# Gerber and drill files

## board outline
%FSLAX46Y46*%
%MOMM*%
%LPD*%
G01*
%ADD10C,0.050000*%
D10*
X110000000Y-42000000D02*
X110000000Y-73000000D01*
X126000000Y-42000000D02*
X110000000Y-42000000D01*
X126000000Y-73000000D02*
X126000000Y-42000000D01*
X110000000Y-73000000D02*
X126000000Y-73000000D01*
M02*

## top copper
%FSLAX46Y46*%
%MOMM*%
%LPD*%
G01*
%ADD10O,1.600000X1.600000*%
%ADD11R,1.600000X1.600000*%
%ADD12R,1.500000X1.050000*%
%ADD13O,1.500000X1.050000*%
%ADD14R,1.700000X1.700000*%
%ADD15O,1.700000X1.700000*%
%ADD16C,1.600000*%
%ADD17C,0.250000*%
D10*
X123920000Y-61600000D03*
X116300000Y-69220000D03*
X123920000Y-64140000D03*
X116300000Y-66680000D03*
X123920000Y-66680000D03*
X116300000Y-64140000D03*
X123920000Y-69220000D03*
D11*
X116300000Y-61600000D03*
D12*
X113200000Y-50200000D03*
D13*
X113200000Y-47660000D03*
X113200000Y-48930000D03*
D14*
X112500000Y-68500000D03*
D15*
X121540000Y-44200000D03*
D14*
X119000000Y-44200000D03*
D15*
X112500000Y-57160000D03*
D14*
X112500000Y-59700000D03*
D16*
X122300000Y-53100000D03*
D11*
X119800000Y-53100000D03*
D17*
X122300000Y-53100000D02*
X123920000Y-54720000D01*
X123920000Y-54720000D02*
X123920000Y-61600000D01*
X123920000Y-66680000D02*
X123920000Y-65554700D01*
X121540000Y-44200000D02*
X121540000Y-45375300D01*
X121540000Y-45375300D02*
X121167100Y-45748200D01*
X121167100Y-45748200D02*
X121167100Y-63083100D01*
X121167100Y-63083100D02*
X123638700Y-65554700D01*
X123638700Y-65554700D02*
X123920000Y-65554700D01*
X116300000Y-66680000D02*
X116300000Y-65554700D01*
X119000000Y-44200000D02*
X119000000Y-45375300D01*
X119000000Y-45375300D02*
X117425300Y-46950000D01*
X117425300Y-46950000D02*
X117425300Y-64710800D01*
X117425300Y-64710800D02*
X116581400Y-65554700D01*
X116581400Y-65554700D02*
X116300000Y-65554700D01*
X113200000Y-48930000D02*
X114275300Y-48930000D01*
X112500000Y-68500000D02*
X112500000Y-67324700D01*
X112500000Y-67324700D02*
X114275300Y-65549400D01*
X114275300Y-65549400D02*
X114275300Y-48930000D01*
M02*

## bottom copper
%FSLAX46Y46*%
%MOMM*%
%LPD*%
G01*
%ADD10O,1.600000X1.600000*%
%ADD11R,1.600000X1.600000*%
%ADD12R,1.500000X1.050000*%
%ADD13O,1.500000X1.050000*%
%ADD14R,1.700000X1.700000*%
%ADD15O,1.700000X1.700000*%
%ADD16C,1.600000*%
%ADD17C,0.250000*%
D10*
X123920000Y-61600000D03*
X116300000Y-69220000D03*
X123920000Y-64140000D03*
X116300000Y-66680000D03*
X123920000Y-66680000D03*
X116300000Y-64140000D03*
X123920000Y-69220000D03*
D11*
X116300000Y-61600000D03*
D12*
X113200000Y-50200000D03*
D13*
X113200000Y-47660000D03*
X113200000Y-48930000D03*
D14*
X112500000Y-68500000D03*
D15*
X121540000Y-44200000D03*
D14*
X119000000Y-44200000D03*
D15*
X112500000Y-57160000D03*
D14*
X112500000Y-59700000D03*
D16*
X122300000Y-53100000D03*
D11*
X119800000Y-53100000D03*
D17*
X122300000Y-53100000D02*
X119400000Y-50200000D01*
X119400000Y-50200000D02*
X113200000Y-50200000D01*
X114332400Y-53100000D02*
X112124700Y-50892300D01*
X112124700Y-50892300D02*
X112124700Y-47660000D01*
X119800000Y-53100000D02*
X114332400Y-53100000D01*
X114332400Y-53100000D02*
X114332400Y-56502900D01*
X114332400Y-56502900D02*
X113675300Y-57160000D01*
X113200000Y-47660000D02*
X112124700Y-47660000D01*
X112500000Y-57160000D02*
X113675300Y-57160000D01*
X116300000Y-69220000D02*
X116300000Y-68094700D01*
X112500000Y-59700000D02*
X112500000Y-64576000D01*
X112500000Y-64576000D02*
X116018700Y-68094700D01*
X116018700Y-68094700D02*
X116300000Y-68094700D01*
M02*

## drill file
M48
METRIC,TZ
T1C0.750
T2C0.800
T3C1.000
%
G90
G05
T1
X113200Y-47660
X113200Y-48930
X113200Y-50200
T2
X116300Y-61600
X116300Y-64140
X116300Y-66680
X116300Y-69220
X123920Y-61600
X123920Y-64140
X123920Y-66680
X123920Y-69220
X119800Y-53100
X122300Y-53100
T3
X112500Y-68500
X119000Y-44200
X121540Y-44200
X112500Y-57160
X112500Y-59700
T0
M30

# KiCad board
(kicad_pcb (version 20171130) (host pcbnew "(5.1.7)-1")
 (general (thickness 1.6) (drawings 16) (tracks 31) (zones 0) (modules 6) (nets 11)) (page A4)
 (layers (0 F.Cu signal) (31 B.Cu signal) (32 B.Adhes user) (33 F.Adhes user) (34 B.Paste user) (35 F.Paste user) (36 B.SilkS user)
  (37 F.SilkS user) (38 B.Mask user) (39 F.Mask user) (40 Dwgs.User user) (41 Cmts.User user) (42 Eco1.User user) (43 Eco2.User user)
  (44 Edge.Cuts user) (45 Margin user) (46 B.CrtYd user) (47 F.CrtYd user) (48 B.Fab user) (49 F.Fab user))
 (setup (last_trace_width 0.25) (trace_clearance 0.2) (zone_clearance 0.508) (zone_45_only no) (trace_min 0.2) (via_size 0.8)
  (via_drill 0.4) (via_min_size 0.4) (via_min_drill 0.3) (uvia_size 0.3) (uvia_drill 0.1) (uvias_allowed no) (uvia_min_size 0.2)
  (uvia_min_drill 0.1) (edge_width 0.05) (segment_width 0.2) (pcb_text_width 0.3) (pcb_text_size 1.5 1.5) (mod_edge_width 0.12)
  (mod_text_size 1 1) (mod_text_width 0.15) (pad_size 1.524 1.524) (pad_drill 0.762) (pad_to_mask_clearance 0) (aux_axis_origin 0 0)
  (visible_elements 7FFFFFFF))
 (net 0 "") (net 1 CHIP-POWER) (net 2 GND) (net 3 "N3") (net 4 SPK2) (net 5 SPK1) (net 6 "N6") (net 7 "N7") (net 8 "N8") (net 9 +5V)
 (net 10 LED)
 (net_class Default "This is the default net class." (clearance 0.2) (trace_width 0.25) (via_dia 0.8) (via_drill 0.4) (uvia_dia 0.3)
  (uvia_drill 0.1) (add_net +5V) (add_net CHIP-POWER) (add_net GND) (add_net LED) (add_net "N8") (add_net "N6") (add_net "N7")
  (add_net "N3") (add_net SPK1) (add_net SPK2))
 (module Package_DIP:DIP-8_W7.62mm (layer F.Cu) (at 116.3 61.6)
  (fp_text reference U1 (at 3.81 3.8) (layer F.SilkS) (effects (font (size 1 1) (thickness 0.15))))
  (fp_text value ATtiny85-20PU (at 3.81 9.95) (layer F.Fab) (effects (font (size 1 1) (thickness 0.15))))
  (pad 8 thru_hole oval (at 7.62 0) (size 1.6 1.6) (drill 0.8) (layers *.Cu *.Mask) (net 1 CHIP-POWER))
  (pad 4 thru_hole oval (at 0 7.62) (size 1.6 1.6) (drill 0.8) (layers *.Cu *.Mask) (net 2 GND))
  (pad 7 thru_hole oval (at 7.62 2.54) (size 1.6 1.6) (drill 0.8) (layers *.Cu *.Mask) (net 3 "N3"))
  (pad 3 thru_hole oval (at 0 5.08) (size 1.6 1.6) (drill 0.8) (layers *.Cu *.Mask) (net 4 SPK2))
  (pad 6 thru_hole oval (at 7.62 5.08) (size 1.6 1.6) (drill 0.8) (layers *.Cu *.Mask) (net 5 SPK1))
  (pad 2 thru_hole oval (at 0 2.54) (size 1.6 1.6) (drill 0.8) (layers *.Cu *.Mask) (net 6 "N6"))
  (pad 5 thru_hole oval (at 7.62 7.62) (size 1.6 1.6) (drill 0.8) (layers *.Cu *.Mask) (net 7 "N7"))
  (pad 1 thru_hole rect (at 0 0) (size 1.6 1.6) (drill 0.8) (layers *.Cu *.Mask) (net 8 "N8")))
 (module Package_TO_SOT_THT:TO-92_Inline (layer F.Cu) (at 113.2 50.2 90)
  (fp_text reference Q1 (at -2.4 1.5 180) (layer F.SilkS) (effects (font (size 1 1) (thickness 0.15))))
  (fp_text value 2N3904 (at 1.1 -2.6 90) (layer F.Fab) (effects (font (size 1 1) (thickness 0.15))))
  (pad 1 thru_hole rect (at 0 0 90) (size 1.05 1.5) (drill 0.75) (layers *.Cu *.Mask) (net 1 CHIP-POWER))
  (pad 3 thru_hole oval (at 2.54 0 90) (size 1.05 1.5) (drill 0.75) (layers *.Cu *.Mask) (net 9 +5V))
  (pad 2 thru_hole oval (at 1.27 0 90) (size 1.05 1.5) (drill 0.75) (layers *.Cu *.Mask) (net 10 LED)))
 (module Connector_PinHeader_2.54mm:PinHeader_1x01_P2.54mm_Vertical (layer F.Cu) (at 112.5 68.5)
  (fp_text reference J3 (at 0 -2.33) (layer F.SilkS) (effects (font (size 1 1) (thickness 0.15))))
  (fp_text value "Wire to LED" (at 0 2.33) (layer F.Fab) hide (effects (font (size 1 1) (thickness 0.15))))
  (pad 1 thru_hole rect (at 0 0) (size 1.7 1.7) (drill 1) (layers *.Cu *.Mask) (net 10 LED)))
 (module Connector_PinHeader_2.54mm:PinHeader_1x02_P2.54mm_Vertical (layer F.Cu) (at 119 44.2 90)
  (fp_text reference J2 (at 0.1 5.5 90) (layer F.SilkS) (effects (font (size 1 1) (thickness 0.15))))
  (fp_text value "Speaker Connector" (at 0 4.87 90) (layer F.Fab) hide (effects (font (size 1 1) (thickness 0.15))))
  (pad 2 thru_hole oval (at 0 2.54 90) (size 1.7 1.7) (drill 1) (layers *.Cu *.Mask) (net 5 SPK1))
  (pad 1 thru_hole rect (at 0 0 90) (size 1.7 1.7) (drill 1) (layers *.Cu *.Mask) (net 4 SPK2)))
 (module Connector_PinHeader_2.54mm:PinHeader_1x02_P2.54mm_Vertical (layer F.Cu) (at 112.5 59.7 180)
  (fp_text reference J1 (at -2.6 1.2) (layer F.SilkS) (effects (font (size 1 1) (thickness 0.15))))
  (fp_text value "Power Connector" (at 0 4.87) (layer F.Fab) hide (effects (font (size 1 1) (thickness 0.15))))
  (pad 2 thru_hole oval (at 0 2.54 180) (size 1.7 1.7) (drill 1) (layers *.Cu *.Mask) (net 9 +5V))
  (pad 1 thru_hole rect (at 0 0 180) (size 1.7 1.7) (drill 1) (layers *.Cu *.Mask) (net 2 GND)))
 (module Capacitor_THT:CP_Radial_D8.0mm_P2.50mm (layer F.Cu) (at 119.8 53.1)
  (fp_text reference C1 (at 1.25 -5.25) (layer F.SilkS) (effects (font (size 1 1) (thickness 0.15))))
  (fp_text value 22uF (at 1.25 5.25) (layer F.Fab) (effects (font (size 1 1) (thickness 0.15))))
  (pad 2 thru_hole circle (at 2.5 0) (size 1.6 1.6) (drill 0.8) (layers *.Cu *.Mask) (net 1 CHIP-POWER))
  (pad 1 thru_hole rect (at 0 0) (size 1.6 1.6) (drill 0.8) (layers *.Cu *.Mask) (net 9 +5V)))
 (gr_line (start 110 42) (end 110 73) (layer Edge.Cuts) (width 0.05))
 (gr_line (start 126 42) (end 110 42) (layer Edge.Cuts) (width 0.05))
 (gr_line (start 126 73) (end 126 42) (layer Edge.Cuts) (width 0.05))
 (gr_line (start 110 73) (end 126 73) (layer Edge.Cuts) (width 0.05))
 (segment (start 122.3 53.1) (end 123.92 54.72) (width 0.25) (layer F.Cu) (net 1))
 (segment (start 123.92 54.72) (end 123.92 61.6) (width 0.25) (layer F.Cu) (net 1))
 (segment (start 122.3 53.1) (end 119.4 50.2) (width 0.25) (layer B.Cu) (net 1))
 (segment (start 119.4 50.2) (end 113.2 50.2) (width 0.25) (layer B.Cu) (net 1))
 (segment (start 114.3324 53.1) (end 112.1247 50.8923) (width 0.25) (layer B.Cu) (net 9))
 (segment (start 112.1247 50.8923) (end 112.1247 47.66) (width 0.25) (layer B.Cu) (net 9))
 (segment (start 119.8 53.1) (end 114.3324 53.1) (width 0.25) (layer B.Cu) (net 9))
 (segment (start 114.3324 53.1) (end 114.3324 56.5029) (width 0.25) (layer B.Cu) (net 9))
 (segment (start 114.3324 56.5029) (end 113.6753 57.16) (width 0.25) (layer B.Cu) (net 9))
 (segment (start 113.2 47.66) (end 112.1247 47.66) (width 0.25) (layer B.Cu) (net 9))
 (segment (start 112.5 57.16) (end 113.6753 57.16) (width 0.25) (layer B.Cu) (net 9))
 (segment (start 116.3 69.22) (end 116.3 68.0947) (width 0.25) (layer B.Cu) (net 2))
 (segment (start 112.5 59.7) (end 112.5 64.576) (width 0.25) (layer B.Cu) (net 2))
 (segment (start 112.5 64.576) (end 116.0187 68.0947) (width 0.25) (layer B.Cu) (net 2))
 (segment (start 116.0187 68.0947) (end 116.3 68.0947) (width 0.25) (layer B.Cu) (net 2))
 (segment (start 123.92 66.68) (end 123.92 65.5547) (width 0.25) (layer F.Cu) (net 5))
 (segment (start 121.54 44.2) (end 121.54 45.3753) (width 0.25) (layer F.Cu) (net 5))
 (segment (start 121.54 45.3753) (end 121.1671 45.7482) (width 0.25) (layer F.Cu) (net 5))
 (segment (start 121.1671 45.7482) (end 121.1671 63.0831) (width 0.25) (layer F.Cu) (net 5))
 (segment (start 121.1671 63.0831) (end 123.6387 65.5547) (width 0.25) (layer F.Cu) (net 5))
 (segment (start 123.6387 65.5547) (end 123.92 65.5547) (width 0.25) (layer F.Cu) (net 5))
 (segment (start 116.3 66.68) (end 116.3 65.5547) (width 0.25) (layer F.Cu) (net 4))
 (segment (start 119 44.2) (end 119 45.3753) (width 0.25) (layer F.Cu) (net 4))
 (segment (start 119 45.3753) (end 117.4253 46.95) (width 0.25) (layer F.Cu) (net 4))
 (segment (start 117.4253 46.95) (end 117.4253 64.7108) (width 0.25) (layer F.Cu) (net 4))
 (segment (start 117.4253 64.7108) (end 116.5814 65.5547) (width 0.25) (layer F.Cu) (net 4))
 (segment (start 116.5814 65.5547) (end 116.3 65.5547) (width 0.25) (layer F.Cu) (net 4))
 (segment (start 113.2 48.93) (end 114.2753 48.93) (width 0.25) (layer F.Cu) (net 10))
 (segment (start 112.5 68.5) (end 112.5 67.3247) (width 0.25) (layer F.Cu) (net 10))
 (segment (start 112.5 67.3247) (end 114.2753 65.5494) (width 0.25) (layer F.Cu) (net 10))
 (segment (start 114.2753 65.5494) (end 114.2753 48.93) (width 0.25) (layer F.Cu) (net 10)))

